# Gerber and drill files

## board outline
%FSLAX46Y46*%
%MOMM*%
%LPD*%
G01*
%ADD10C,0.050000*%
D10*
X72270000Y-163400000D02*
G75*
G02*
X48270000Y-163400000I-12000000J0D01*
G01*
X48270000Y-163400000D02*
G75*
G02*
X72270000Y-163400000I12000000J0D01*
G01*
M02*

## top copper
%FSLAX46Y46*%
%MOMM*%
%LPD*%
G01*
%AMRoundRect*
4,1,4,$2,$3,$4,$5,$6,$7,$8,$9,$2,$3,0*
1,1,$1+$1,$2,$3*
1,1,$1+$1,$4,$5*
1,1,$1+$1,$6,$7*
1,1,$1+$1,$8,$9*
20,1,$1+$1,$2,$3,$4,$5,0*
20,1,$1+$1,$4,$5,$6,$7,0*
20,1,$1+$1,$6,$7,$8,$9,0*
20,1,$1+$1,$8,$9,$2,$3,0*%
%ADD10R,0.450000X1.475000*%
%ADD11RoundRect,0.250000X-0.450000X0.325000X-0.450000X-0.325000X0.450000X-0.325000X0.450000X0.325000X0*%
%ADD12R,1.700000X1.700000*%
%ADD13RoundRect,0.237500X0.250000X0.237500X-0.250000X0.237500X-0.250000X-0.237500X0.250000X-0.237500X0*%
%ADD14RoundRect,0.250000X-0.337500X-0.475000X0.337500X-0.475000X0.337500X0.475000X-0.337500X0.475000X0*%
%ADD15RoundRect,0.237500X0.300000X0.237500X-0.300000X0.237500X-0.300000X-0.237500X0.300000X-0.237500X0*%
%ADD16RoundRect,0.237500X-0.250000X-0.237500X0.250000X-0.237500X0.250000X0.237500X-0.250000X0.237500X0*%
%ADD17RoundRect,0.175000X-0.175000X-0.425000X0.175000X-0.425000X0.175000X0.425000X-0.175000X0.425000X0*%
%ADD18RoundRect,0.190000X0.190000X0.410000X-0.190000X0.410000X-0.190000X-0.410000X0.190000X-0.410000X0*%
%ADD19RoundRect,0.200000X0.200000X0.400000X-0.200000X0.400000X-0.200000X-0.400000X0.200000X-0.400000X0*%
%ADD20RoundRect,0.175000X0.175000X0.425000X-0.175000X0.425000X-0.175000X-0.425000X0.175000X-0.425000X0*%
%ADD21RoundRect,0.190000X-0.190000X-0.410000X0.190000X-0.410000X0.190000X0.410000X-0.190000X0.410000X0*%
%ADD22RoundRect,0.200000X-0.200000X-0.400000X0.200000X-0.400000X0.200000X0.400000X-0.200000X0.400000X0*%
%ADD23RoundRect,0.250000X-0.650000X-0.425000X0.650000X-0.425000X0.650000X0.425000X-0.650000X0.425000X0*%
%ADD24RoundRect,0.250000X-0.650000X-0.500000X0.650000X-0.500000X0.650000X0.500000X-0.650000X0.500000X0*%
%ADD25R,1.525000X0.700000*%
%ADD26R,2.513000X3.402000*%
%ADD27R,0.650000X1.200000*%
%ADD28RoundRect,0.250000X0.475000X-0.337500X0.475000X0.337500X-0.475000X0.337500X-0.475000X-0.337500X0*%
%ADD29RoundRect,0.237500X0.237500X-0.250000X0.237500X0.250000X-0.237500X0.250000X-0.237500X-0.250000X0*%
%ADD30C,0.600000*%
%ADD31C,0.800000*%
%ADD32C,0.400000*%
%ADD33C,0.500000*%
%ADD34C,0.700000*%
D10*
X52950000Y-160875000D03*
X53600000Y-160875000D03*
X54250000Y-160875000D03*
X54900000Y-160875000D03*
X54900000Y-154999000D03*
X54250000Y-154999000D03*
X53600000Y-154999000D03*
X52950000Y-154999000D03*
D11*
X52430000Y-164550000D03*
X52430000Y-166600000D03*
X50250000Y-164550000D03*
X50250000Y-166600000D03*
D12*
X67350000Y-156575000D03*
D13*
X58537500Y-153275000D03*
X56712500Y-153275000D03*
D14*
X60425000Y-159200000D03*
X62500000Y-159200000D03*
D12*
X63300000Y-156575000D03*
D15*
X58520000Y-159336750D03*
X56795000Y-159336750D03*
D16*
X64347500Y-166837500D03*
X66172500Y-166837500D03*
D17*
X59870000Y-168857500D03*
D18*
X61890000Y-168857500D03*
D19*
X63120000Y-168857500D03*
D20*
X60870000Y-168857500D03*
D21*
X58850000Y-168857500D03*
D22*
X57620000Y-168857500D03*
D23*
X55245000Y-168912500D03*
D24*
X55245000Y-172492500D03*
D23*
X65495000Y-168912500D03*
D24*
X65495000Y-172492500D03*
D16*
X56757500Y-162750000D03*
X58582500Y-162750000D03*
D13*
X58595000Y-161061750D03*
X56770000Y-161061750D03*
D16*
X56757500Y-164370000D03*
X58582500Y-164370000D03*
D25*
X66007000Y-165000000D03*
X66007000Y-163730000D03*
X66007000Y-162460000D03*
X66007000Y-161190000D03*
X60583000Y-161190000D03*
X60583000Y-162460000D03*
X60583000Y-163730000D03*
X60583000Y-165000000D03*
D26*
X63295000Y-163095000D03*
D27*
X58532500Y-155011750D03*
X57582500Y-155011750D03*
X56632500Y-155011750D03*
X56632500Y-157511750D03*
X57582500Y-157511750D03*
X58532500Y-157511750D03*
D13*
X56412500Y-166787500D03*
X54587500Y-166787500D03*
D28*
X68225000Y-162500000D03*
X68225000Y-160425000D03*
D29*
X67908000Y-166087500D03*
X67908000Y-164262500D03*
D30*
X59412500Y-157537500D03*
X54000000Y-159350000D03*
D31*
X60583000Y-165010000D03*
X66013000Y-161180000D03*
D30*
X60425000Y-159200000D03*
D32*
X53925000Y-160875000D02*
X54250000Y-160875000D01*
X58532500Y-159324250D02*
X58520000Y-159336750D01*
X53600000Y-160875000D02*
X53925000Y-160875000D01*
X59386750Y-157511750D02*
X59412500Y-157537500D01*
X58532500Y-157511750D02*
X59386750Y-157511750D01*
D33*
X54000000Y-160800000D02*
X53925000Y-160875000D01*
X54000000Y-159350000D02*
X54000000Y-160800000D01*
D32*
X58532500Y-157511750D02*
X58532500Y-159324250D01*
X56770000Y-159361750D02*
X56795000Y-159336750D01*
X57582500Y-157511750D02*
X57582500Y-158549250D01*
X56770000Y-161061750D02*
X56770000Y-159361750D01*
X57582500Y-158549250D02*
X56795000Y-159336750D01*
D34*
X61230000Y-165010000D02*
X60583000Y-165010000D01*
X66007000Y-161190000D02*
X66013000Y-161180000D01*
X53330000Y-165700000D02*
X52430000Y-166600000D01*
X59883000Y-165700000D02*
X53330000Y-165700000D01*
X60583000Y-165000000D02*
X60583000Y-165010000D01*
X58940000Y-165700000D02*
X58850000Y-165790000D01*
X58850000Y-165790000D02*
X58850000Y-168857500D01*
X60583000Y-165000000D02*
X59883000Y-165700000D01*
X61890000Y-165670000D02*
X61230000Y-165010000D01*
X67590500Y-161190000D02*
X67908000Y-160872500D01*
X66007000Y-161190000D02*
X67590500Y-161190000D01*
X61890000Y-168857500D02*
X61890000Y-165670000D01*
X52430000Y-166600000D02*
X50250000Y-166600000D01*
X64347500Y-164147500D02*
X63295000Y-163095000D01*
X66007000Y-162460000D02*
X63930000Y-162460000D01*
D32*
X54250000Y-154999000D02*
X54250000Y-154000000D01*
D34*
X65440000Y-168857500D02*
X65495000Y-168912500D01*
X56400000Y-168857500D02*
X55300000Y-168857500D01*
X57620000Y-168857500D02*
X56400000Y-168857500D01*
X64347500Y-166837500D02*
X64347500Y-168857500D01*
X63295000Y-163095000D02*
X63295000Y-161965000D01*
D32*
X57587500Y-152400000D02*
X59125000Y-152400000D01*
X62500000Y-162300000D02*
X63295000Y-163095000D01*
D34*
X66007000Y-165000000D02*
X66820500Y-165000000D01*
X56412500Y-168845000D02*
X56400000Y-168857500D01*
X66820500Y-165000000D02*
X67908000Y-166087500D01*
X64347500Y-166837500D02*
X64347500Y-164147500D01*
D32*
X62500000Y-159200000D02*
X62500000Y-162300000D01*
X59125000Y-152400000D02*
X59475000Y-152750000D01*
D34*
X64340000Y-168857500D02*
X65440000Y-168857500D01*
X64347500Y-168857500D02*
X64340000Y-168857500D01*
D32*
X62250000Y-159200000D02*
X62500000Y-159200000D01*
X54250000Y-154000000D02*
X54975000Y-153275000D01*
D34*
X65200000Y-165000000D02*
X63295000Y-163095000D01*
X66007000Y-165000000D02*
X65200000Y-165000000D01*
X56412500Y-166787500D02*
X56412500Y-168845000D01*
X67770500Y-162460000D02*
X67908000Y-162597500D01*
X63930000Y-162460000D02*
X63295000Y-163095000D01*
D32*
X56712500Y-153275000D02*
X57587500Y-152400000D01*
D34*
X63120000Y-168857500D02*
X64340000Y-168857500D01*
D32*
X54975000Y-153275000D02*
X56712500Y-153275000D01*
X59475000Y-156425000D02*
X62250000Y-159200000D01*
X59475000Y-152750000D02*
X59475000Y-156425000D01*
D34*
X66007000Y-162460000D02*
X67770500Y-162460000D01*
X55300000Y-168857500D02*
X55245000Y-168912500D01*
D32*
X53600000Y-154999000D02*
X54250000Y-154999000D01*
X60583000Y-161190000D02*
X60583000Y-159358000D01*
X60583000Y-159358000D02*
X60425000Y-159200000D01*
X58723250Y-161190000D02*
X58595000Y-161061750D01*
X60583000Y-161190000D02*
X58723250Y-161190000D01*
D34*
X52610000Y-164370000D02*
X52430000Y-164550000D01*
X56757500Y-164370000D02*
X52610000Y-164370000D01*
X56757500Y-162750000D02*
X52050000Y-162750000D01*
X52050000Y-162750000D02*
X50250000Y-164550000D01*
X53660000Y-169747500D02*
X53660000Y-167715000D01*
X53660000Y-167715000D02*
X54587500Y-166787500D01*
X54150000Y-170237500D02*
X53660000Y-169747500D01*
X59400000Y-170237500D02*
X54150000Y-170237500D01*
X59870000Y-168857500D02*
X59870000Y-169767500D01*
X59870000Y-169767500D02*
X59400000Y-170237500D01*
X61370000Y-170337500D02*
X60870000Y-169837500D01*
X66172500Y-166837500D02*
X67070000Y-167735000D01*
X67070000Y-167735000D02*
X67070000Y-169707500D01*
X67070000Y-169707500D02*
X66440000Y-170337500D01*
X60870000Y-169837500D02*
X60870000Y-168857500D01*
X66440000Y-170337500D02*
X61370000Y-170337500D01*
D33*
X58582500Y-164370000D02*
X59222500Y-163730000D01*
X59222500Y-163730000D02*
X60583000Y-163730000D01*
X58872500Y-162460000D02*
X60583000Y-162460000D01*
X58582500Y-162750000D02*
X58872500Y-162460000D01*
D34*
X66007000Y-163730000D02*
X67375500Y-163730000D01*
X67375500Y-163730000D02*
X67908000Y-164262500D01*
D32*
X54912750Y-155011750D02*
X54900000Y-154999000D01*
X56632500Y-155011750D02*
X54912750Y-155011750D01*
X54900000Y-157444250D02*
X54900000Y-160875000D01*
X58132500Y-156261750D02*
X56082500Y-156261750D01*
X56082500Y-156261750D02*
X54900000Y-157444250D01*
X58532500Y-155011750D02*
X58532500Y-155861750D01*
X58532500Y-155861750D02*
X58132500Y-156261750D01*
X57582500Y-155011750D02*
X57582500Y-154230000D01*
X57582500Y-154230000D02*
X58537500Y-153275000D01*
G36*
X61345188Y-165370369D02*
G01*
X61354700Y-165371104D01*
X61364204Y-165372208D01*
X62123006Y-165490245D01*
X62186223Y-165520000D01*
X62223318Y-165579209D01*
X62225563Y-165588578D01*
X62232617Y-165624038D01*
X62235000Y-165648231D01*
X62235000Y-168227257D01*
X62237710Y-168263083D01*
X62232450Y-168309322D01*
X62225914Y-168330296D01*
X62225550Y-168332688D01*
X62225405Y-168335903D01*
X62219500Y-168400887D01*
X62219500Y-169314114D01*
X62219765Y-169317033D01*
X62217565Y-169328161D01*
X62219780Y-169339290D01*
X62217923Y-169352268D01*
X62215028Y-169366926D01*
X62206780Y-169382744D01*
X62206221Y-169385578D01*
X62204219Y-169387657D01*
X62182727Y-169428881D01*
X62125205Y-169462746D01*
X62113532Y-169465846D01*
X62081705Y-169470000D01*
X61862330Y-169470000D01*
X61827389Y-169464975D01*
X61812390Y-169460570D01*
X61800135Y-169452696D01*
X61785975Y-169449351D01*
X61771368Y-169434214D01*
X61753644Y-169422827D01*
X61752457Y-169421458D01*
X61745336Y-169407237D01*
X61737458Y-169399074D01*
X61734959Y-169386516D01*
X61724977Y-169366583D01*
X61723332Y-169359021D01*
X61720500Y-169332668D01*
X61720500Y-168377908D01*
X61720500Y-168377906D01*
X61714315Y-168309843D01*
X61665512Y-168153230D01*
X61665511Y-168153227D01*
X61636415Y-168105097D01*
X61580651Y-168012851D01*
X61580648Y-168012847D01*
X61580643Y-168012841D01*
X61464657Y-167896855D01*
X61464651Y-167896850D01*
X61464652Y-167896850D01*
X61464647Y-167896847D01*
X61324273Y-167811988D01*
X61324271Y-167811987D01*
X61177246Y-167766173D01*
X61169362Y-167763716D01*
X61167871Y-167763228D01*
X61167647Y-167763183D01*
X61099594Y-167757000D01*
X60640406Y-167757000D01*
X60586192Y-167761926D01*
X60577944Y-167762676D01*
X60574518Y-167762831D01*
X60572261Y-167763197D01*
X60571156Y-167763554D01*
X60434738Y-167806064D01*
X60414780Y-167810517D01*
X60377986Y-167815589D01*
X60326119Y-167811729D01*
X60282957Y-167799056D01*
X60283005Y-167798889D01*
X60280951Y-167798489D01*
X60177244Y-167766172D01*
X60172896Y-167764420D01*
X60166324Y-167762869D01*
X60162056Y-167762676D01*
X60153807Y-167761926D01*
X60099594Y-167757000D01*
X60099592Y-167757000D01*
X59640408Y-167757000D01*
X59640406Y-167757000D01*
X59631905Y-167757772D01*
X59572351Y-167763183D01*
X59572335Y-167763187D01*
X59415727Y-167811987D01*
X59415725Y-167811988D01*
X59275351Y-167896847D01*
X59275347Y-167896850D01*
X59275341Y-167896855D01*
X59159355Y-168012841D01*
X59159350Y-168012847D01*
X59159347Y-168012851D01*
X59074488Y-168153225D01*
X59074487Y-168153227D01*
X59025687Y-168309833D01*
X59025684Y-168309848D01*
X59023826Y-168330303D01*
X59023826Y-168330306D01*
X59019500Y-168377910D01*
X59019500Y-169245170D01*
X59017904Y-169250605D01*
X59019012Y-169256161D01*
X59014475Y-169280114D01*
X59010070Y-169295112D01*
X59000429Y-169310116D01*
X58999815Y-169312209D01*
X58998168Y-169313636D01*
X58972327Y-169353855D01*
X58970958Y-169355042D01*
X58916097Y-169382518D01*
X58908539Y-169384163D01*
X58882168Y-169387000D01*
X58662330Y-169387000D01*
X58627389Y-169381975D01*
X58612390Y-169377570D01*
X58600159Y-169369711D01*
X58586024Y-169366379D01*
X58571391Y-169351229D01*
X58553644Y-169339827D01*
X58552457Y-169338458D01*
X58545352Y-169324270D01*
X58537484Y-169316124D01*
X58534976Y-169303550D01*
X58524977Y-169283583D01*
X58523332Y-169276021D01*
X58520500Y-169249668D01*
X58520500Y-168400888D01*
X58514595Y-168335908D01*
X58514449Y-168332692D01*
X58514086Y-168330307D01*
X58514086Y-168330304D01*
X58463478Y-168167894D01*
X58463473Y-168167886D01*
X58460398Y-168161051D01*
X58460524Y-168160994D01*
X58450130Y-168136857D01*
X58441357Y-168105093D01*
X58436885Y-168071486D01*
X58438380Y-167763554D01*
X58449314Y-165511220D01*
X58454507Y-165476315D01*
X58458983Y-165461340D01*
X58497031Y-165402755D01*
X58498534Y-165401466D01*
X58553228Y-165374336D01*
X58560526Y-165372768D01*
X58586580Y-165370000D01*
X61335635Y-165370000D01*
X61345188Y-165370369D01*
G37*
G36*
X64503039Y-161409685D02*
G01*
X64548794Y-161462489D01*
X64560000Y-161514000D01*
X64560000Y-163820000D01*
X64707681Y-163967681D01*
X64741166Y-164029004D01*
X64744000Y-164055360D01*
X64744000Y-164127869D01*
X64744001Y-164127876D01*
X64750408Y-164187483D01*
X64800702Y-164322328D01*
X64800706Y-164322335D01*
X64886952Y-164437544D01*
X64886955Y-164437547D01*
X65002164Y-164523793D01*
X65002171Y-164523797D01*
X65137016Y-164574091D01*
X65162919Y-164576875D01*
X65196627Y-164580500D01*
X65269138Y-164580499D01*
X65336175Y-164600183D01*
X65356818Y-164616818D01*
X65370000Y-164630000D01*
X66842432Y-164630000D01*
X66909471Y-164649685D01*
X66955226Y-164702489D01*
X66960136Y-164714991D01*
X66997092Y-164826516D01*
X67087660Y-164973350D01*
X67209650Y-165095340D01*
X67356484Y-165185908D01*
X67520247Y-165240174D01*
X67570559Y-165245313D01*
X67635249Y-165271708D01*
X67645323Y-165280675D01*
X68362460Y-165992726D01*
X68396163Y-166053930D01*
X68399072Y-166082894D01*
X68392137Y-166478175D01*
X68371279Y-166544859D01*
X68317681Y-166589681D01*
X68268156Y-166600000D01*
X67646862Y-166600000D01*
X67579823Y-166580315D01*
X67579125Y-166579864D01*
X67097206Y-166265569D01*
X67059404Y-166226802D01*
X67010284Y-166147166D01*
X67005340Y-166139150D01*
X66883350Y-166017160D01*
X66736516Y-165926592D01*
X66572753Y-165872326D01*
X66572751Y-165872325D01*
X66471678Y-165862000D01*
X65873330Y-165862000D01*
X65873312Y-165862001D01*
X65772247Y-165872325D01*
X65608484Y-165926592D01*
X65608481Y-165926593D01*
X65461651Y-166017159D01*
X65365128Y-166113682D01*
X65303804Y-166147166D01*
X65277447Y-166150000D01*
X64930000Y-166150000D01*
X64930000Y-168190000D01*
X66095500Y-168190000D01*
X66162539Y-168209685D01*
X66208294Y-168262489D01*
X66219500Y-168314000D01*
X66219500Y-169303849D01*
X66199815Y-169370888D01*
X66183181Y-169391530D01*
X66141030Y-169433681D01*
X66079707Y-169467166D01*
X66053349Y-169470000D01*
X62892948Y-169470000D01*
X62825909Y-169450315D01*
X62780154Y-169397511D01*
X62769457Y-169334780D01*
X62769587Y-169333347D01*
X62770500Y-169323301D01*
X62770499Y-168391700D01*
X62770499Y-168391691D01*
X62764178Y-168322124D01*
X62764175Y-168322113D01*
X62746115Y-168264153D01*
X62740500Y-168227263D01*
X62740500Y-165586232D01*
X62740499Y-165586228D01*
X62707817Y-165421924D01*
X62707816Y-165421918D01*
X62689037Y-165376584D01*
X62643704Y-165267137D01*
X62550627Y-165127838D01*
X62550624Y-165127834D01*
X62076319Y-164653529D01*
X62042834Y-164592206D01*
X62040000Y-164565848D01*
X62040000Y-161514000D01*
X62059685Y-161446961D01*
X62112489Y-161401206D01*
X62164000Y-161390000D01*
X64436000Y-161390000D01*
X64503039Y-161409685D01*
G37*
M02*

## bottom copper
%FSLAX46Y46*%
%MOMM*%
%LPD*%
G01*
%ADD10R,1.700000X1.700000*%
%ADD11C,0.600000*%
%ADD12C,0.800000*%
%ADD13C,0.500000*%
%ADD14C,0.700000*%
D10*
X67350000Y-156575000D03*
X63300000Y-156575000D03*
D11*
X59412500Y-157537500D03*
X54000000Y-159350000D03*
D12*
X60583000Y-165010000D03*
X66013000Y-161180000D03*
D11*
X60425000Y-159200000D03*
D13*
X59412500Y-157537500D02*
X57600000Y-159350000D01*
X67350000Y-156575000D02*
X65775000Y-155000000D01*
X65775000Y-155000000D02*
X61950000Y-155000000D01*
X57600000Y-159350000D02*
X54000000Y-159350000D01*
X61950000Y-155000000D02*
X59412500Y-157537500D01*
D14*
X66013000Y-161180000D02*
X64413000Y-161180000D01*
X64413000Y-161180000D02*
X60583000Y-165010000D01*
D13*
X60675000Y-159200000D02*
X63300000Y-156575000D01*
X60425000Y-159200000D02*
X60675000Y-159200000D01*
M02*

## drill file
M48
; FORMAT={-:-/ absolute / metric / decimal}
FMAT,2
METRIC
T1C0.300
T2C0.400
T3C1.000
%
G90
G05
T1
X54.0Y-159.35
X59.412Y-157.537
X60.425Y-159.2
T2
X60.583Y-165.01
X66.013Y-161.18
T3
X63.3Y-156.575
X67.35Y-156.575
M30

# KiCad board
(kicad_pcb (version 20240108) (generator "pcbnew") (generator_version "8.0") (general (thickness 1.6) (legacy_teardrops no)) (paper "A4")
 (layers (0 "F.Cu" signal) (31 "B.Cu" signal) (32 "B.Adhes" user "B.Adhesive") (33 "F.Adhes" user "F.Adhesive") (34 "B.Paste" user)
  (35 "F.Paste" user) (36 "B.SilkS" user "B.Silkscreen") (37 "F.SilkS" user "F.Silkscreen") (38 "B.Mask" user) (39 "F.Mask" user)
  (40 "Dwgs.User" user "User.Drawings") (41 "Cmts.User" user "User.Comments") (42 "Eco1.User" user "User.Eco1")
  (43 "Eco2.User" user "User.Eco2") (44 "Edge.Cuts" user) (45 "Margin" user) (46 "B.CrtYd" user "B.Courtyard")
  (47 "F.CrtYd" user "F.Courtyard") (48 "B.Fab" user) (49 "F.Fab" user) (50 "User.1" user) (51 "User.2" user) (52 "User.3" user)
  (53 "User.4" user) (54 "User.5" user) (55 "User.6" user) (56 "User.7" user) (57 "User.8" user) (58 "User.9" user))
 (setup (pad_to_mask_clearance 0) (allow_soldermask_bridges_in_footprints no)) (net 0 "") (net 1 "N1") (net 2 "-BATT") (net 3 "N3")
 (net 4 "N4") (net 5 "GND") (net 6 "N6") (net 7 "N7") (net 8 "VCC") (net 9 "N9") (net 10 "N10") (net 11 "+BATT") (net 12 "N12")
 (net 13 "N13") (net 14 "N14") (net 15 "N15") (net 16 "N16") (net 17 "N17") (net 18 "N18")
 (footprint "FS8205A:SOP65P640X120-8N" (layer "F.Cu") (at 53.925 157.937 90)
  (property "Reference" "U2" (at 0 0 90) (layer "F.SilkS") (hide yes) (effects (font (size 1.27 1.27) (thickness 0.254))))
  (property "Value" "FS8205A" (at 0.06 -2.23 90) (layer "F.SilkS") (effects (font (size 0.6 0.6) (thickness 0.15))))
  (pad "1" smd rect (at -2.938 -0.975 180) (size 0.45 1.475) (layers "F.Cu" "F.Paste" "F.Mask") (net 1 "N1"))
  (pad "2" smd rect (at -2.938 -0.325 180) (size 0.45 1.475) (layers "F.Cu" "F.Paste" "F.Mask") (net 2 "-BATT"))
  (pad "3" smd rect (at -2.938 0.325 180) (size 0.45 1.475) (layers "F.Cu" "F.Paste" "F.Mask") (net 2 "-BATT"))
  (pad "4" smd rect (at -2.938 0.975 180) (size 0.45 1.475) (layers "F.Cu" "F.Paste" "F.Mask") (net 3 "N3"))
  (pad "5" smd rect (at 2.938 0.975 180) (size 0.45 1.475) (layers "F.Cu" "F.Paste" "F.Mask") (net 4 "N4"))
  (pad "6" smd rect (at 2.938 0.325 180) (size 0.45 1.475) (layers "F.Cu" "F.Paste" "F.Mask") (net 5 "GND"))
  (pad "7" smd rect (at 2.938 -0.325 180) (size 0.45 1.475) (layers "F.Cu" "F.Paste" "F.Mask") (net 5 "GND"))
  (pad "8" smd rect (at 2.938 -0.975 180) (size 0.45 1.475) (layers "F.Cu" "F.Paste" "F.Mask") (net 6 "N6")))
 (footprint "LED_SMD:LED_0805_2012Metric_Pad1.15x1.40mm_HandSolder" (layer "F.Cu") (at 52.43 165.575 -90)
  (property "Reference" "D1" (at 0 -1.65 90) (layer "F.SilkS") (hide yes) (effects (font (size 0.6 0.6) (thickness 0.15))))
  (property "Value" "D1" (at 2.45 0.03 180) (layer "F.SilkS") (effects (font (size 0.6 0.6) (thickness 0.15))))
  (pad "1" smd roundrect (at -1.025 0 270) (size 1.15 1.4) (layers "F.Cu" "F.Paste" "F.Mask") (roundrect_rratio 0.2173913043) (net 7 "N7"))
  (pad "2" smd roundrect (at 1.025 0 270) (size 1.15 1.4) (layers "F.Cu" "F.Paste" "F.Mask") (roundrect_rratio 0.2173913043) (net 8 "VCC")))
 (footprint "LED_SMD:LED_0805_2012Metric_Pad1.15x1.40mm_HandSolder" (layer "F.Cu") (at 50.25 165.575 -90)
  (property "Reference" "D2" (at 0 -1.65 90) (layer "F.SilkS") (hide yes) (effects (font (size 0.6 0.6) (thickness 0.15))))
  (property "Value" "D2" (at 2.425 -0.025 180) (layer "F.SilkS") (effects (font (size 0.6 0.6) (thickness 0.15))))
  (pad "1" smd roundrect (at -1.025 0 270) (size 1.15 1.4) (layers "F.Cu" "F.Paste" "F.Mask") (roundrect_rratio 0.2173913043) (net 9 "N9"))
  (pad "2" smd roundrect (at 1.025 0 270) (size 1.15 1.4) (layers "F.Cu" "F.Paste" "F.Mask") (roundrect_rratio 0.2173913043) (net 8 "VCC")))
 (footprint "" (layer "F.Cu") (at 67.35 156.575)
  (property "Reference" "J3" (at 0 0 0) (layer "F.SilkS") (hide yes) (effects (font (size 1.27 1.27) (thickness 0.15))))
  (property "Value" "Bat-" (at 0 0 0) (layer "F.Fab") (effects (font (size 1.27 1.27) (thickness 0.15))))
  (pad "1" thru_hole rect (at 0 0 90) (size 1.7 1.7) (drill 1) (layers "*.Cu" "*.Mask") (remove_unused_layers no) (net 2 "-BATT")))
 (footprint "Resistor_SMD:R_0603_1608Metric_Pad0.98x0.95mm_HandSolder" (layer "F.Cu") (at 57.625 153.275 180)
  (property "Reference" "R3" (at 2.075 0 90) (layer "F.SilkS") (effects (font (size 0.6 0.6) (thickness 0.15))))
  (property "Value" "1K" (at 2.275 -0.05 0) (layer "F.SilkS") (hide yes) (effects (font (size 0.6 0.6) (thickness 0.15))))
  (pad "1" smd roundrect (at -0.9125 0 180) (size 0.975 0.95) (layers "F.Cu" "F.Paste" "F.Mask") (roundrect_rratio 0.25) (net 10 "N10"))
  (pad "2" smd roundrect (at 0.9125 0 180) (size 0.975 0.95) (layers "F.Cu" "F.Paste" "F.Mask") (roundrect_rratio 0.25) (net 5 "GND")))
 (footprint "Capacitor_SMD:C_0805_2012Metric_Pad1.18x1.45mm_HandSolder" (layer "F.Cu") (at 61.4625 159.2)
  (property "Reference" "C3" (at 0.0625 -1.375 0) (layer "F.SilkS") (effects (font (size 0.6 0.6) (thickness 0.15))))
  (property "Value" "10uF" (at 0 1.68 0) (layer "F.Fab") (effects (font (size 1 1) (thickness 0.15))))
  (pad "1" smd roundrect (at -1.0375 0) (size 1.175 1.45) (layers "F.Cu" "F.Paste" "F.Mask") (roundrect_rratio 0.212766) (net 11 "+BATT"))
  (pad "2" smd roundrect (at 1.0375 0) (size 1.175 1.45) (layers "F.Cu" "F.Paste" "F.Mask") (roundrect_rratio 0.212766) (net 5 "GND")))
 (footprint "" (layer "F.Cu") (at 63.3 156.575)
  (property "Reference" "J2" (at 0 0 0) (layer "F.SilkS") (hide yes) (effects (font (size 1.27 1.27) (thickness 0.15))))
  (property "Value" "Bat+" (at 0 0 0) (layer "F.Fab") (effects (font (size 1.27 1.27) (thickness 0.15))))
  (pad "1" thru_hole rect (at 0 0 90) (size 1.7 1.7) (drill 1) (layers "*.Cu" "*.Mask") (remove_unused_layers no) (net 11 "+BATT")))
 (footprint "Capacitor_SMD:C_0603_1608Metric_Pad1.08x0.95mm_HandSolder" (layer "F.Cu") (at 57.6575 159.33675 180)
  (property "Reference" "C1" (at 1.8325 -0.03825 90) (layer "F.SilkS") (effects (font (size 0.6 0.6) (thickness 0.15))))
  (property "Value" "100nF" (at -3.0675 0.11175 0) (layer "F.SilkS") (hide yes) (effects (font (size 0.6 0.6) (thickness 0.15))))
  (pad "1" smd roundrect (at -0.8625 0 180) (size 1.075 0.95) (layers "F.Cu" "F.Paste" "F.Mask") (roundrect_rratio 0.25) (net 2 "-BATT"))
  (pad "2" smd roundrect (at 0.8625 0 180) (size 1.075 0.95) (layers "F.Cu" "F.Paste" "F.Mask") (roundrect_rratio 0.25) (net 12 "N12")))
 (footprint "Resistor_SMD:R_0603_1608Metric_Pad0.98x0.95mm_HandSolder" (layer "F.Cu") (at 65.26 166.8375)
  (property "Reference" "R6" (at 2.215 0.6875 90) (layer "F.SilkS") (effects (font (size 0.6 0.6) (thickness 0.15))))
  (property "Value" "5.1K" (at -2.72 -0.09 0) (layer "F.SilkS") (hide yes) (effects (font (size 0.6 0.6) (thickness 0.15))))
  (pad "1" smd roundrect (at -0.9125 0) (size 0.975 0.95) (layers "F.Cu" "F.Paste" "F.Mask") (roundrect_rratio 0.25) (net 5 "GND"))
  (pad "2" smd roundrect (at 0.9125 0) (size 0.975 0.95) (layers "F.Cu" "F.Paste" "F.Mask") (roundrect_rratio 0.25) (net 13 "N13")))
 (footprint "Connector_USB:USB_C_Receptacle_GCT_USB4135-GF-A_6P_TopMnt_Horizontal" (layer "F.Cu") (at 60.37 171.89)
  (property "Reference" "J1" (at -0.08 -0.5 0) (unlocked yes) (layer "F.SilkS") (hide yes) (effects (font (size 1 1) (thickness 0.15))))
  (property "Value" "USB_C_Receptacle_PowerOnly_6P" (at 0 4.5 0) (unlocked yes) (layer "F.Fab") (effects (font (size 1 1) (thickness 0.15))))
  (pad "A5" smd roundrect (at -0.5 -3.0325) (size 0.7 1.2) (layers "F.Cu" "F.Paste" "F.Mask") (roundrect_rratio 0.25) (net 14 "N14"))
  (pad "A9" smd roundrect (at 1.52 -3.0325 180) (size 0.76 1.2) (layers "F.Cu" "F.Paste" "F.Mask") (roundrect_rratio 0.25) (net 8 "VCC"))
  (pad "A12" smd roundrect (at 2.75 -3.0325 180) (size 0.8 1.2) (layers "F.Cu" "F.Paste" "F.Mask") (roundrect_rratio 0.25) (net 5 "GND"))
  (pad "B5" smd roundrect (at 0.5 -3.0325 180) (size 0.7 1.2) (layers "F.Cu" "F.Paste" "F.Mask") (roundrect_rratio 0.25) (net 13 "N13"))
  (pad "B9" smd roundrect (at -1.52 -3.0325) (size 0.76 1.2) (layers "F.Cu" "F.Paste" "F.Mask") (roundrect_rratio 0.25) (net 8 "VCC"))
  (pad "B12" smd roundrect (at -2.75 -3.0325) (size 0.8 1.2) (layers "F.Cu" "F.Paste" "F.Mask") (roundrect_rratio 0.25) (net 5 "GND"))
  (pad "S1" smd roundrect (at -5.125 -2.9775) (size 1.8 1.35) (layers "F.Cu" "F.Paste" "F.Mask") (roundrect_rratio 0.1851851852)
   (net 5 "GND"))
  (pad "S1" smd roundrect (at -5.125 0.6025) (size 1.8 1.5) (layers "F.Cu" "F.Paste" "F.Mask") (roundrect_rratio 0.1666666667) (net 5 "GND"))
  (pad "S1" smd roundrect (at 5.125 -2.9775) (size 1.8 1.35) (layers "F.Cu" "F.Paste" "F.Mask") (roundrect_rratio 0.1851851852)
   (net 5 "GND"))
  (pad "S1" smd roundrect (at 5.125 0.6025) (size 1.8 1.5) (layers "F.Cu" "F.Paste" "F.Mask") (roundrect_rratio 0.1666666667) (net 5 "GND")))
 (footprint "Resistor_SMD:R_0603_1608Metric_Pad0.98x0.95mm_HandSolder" (layer "F.Cu") (at 57.67 162.75)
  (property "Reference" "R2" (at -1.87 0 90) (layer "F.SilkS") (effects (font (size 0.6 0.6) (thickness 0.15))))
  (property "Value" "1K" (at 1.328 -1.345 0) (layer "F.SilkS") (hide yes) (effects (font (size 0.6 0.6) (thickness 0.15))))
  (pad "1" smd roundrect (at -0.9125 0) (size 0.975 0.95) (layers "F.Cu" "F.Paste" "F.Mask") (roundrect_rratio 0.25) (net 9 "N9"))
  (pad "2" smd roundrect (at 0.9125 0) (size 0.975 0.95) (layers "F.Cu" "F.Paste" "F.Mask") (roundrect_rratio 0.25) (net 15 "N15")))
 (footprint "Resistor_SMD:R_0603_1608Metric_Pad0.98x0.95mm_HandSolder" (layer "F.Cu") (at 57.6825 161.06175 180)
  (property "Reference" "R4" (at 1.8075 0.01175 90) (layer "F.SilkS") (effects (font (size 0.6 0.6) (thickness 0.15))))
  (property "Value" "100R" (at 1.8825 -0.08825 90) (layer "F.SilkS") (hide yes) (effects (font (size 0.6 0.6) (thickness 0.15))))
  (pad "1" smd roundrect (at -0.9125 0 180) (size 0.975 0.95) (layers "F.Cu" "F.Paste" "F.Mask") (roundrect_rratio 0.25) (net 11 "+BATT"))
  (pad "2" smd roundrect (at 0.9125 0 180) (size 0.975 0.95) (layers "F.Cu" "F.Paste" "F.Mask") (roundrect_rratio 0.25) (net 12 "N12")))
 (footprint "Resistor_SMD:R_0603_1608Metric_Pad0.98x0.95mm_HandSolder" (layer "F.Cu") (at 57.67 164.37)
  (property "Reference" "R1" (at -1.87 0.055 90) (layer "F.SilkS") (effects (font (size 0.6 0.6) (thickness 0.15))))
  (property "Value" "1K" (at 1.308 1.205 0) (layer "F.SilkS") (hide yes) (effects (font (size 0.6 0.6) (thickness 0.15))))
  (pad "1" smd roundrect (at -0.9125 0) (size 0.975 0.95) (layers "F.Cu" "F.Paste" "F.Mask") (roundrect_rratio 0.25) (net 7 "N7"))
  (pad "2" smd roundrect (at 0.9125 0) (size 0.975 0.95) (layers "F.Cu" "F.Paste" "F.Mask") (roundrect_rratio 0.25) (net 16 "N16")))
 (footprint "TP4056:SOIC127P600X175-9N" (layer "F.Cu") (at 63.295 163.095 180)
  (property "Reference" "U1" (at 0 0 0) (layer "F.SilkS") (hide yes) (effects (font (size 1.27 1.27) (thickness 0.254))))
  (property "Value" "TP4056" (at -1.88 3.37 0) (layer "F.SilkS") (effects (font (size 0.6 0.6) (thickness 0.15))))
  (pad "1" smd rect (at -2.712 -1.905 270) (size 0.7 1.525) (layers "F.Cu" "F.Paste" "F.Mask") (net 5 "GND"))
  (pad "2" smd rect (at -2.712 -0.635 270) (size 0.7 1.525) (layers "F.Cu" "F.Paste" "F.Mask") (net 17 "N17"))
  (pad "3" smd rect (at -2.712 0.635 270) (size 0.7 1.525) (layers "F.Cu" "F.Paste" "F.Mask") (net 5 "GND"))
  (pad "4" smd rect (at -2.712 1.905 270) (size 0.7 1.525) (layers "F.Cu" "F.Paste" "F.Mask") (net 8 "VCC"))
  (pad "5" smd rect (at 2.712 1.905 270) (size 0.7 1.525) (layers "F.Cu" "F.Paste" "F.Mask") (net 11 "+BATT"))
  (pad "6" smd rect (at 2.712 0.635 270) (size 0.7 1.525) (layers "F.Cu" "F.Paste" "F.Mask") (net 15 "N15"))
  (pad "7" smd rect (at 2.712 -0.635 270) (size 0.7 1.525) (layers "F.Cu" "F.Paste" "F.Mask") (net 16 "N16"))
  (pad "8" smd rect (at 2.712 -1.905 270) (size 0.7 1.525) (layers "F.Cu" "F.Paste" "F.Mask") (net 8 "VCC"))
  (pad "9" smd rect (at 0 0 180) (size 2.513 3.402) (layers "F.Cu" "F.Paste" "F.Mask") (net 5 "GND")))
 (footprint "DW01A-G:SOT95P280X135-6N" (layer "F.Cu") (at 57.5825 156.26175 -90)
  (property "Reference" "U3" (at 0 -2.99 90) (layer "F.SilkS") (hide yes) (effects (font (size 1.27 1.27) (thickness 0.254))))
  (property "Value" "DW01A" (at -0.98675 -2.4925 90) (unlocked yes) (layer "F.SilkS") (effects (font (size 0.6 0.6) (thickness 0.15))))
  (pad "1" smd rect (at -1.25 -0.95) (size 0.65 1.2) (layers "F.Cu" "F.Paste" "F.Mask") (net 3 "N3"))
  (pad "2" smd rect (at -1.25 0) (size 0.65 1.2) (layers "F.Cu" "F.Paste" "F.Mask") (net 10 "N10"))
  (pad "3" smd rect (at -1.25 0.95) (size 0.65 1.2) (layers "F.Cu" "F.Paste" "F.Mask") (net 4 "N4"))
  (pad "4" smd rect (at 1.25 0.95) (size 0.65 1.2) (layers "F.Cu" "F.Paste" "F.Mask") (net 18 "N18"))
  (pad "5" smd rect (at 1.25 0) (size 0.65 1.2) (layers "F.Cu" "F.Paste" "F.Mask") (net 12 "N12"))
  (pad "6" smd rect (at 1.25 -0.95) (size 0.65 1.2) (layers "F.Cu" "F.Paste" "F.Mask") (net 2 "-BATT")))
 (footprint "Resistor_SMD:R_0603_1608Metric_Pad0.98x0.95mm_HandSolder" (layer "F.Cu") (at 55.5 166.7875 180)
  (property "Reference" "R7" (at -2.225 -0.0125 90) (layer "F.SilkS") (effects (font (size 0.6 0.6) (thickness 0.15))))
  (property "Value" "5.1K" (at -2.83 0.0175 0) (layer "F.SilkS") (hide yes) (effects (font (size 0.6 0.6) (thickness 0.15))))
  (pad "1" smd roundrect (at -0.9125 0 180) (size 0.975 0.95) (layers "F.Cu" "F.Paste" "F.Mask") (roundrect_rratio 0.25) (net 5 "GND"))
  (pad "2" smd roundrect (at 0.9125 0 180) (size 0.975 0.95) (layers "F.Cu" "F.Paste" "F.Mask") (roundrect_rratio 0.25) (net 14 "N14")))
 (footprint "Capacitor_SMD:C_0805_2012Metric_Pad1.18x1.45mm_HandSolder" (layer "F.Cu") (at 68.225 161.4625 90)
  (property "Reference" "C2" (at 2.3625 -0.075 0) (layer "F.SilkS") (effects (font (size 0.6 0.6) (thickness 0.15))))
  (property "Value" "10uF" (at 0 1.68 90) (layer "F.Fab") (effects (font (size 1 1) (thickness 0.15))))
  (pad "1" smd roundrect (at -1.0375 0 90) (size 1.175 1.45) (layers "F.Cu" "F.Paste" "F.Mask") (roundrect_rratio 0.212766) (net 5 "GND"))
  (pad "2" smd roundrect (at 1.0375 0 90) (size 1.175 1.45) (layers "F.Cu" "F.Paste" "F.Mask") (roundrect_rratio 0.212766) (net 8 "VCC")))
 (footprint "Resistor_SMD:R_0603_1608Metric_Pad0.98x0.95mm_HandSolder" (layer "F.Cu") (at 67.908 165.175 90)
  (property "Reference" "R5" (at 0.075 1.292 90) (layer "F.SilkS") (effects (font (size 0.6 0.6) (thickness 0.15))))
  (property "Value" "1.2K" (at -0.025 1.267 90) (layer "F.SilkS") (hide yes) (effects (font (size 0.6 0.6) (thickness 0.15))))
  (pad "1" smd roundrect (at -0.9125 0 90) (size 0.975 0.95) (layers "F.Cu" "F.Paste" "F.Mask") (roundrect_rratio 0.25) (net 5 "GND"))
  (pad "2" smd roundrect (at 0.9125 0 90) (size 0.975 0.95) (layers "F.Cu" "F.Paste" "F.Mask") (roundrect_rratio 0.25) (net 17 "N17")))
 (gr_circle (center 60.27 163.4) (end 72.27 163.4) (stroke (width 0.05) (type default)) (fill none) (layer "Edge.Cuts"))
 (segment (start 53.925 160.875) (end 54.25 160.875) (width 0.4) (layer "F.Cu") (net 2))
 (segment (start 58.5325 159.32425) (end 58.52 159.33675) (width 0.4) (layer "F.Cu") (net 2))
 (segment (start 53.6 160.875) (end 53.925 160.875) (width 0.4) (layer "F.Cu") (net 2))
 (segment (start 59.38675 157.51175) (end 59.4125 157.5375) (width 0.4) (layer "F.Cu") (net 2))
 (segment (start 58.5325 157.51175) (end 59.38675 157.51175) (width 0.4) (layer "F.Cu") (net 2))
 (segment (start 54 160.8) (end 53.925 160.875) (width 0.5) (layer "F.Cu") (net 2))
 (segment (start 54 159.35) (end 54 160.8) (width 0.5) (layer "F.Cu") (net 2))
 (segment (start 58.5325 157.51175) (end 58.5325 159.32425) (width 0.4) (layer "F.Cu") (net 2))
 (via (at 59.4125 157.5375) (size 0.6) (drill 0.3) (layers "F.Cu" "B.Cu") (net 2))
 (via (at 54 159.35) (size 0.6) (drill 0.3) (layers "F.Cu" "B.Cu") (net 2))
 (segment (start 59.4125 157.5375) (end 57.6 159.35) (width 0.5) (layer "B.Cu") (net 2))
 (segment (start 67.35 156.575) (end 65.775 155) (width 0.5) (layer "B.Cu") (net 2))
 (segment (start 65.775 155) (end 61.95 155) (width 0.5) (layer "B.Cu") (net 2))
 (segment (start 57.6 159.35) (end 54 159.35) (width 0.5) (layer "B.Cu") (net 2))
 (segment (start 61.95 155) (end 59.4125 157.5375) (width 0.5) (layer "B.Cu") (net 2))
 (segment (start 56.77 159.36175) (end 56.795 159.33675) (width 0.4) (layer "F.Cu") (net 12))
 (segment (start 57.5825 157.51175) (end 57.5825 158.54925) (width 0.4) (layer "F.Cu") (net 12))
 (segment (start 56.77 161.06175) (end 56.77 159.36175) (width 0.4) (layer "F.Cu") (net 12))
 (segment (start 57.5825 158.54925) (end 56.795 159.33675) (width 0.4) (layer "F.Cu") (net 12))
 (segment (start 61.23 165.01) (end 60.583 165.01) (width 0.7) (layer "F.Cu") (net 8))
 (segment (start 66.007 161.19) (end 66.013 161.18) (width 0.7) (layer "F.Cu") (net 8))
 (segment (start 53.33 165.7) (end 52.43 166.6) (width 0.7) (layer "F.Cu") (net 8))
 (segment (start 59.883 165.7) (end 53.33 165.7) (width 0.7) (layer "F.Cu") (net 8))
 (segment (start 60.583 165) (end 60.583 165.01) (width 0.7) (layer "F.Cu") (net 8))
 (segment (start 58.94 165.7) (end 58.85 165.79) (width 0.7) (layer "F.Cu") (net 8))
 (segment (start 58.85 165.79) (end 58.85 168.8575) (width 0.7) (layer "F.Cu") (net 8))
 (segment (start 60.583 165) (end 59.883 165.7) (width 0.7) (layer "F.Cu") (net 8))
 (segment (start 61.89 165.67) (end 61.23 165.01) (width 0.7) (layer "F.Cu") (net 8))
 (segment (start 67.5905 161.19) (end 67.908 160.8725) (width 0.7) (layer "F.Cu") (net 8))
 (segment (start 66.007 161.19) (end 67.5905 161.19) (width 0.7) (layer "F.Cu") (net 8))
 (segment (start 61.89 168.8575) (end 61.89 165.67) (width 0.7) (layer "F.Cu") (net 8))
 (segment (start 52.43 166.6) (end 50.25 166.6) (width 0.7) (layer "F.Cu") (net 8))
 (via (at 60.583 165.01) (size 0.8) (drill 0.4) (layers "F.Cu" "B.Cu") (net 8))
 (via (at 66.013 161.18) (size 0.8) (drill 0.4) (layers "F.Cu" "B.Cu") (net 8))
 (segment (start 66.013 161.18) (end 64.413 161.18) (width 0.7) (layer "B.Cu") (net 8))
 (segment (start 64.413 161.18) (end 60.583 165.01) (width 0.7) (layer "B.Cu") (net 8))
 (segment (start 64.3475 164.1475) (end 63.295 163.095) (width 0.7) (layer "F.Cu") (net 5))
 (segment (start 66.007 162.46) (end 63.93 162.46) (width 0.7) (layer "F.Cu") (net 5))
 (segment (start 54.25 154.999) (end 54.25 154) (width 0.4) (layer "F.Cu") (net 5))
 (segment (start 65.44 168.8575) (end 65.495 168.9125) (width 0.7) (layer "F.Cu") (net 5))
 (segment (start 56.4 168.8575) (end 55.3 168.8575) (width 0.7) (layer "F.Cu") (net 5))
 (segment (start 57.62 168.8575) (end 56.4 168.8575) (width 0.7) (layer "F.Cu") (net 5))
 (segment (start 64.3475 166.8375) (end 64.3475 168.8575) (width 0.7) (layer "F.Cu") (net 5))
 (segment (start 63.295 163.095) (end 63.295 161.965) (width 0.7) (layer "F.Cu") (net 5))
 (segment (start 57.5875 152.4) (end 59.125 152.4) (width 0.4) (layer "F.Cu") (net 5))
 (segment (start 62.5 162.3) (end 63.295 163.095) (width 0.4) (layer "F.Cu") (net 5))
 (segment (start 66.007 165) (end 66.8205 165) (width 0.7) (layer "F.Cu") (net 5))
 (segment (start 56.4125 168.845) (end 56.4 168.8575) (width 0.7) (layer "F.Cu") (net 5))
 (segment (start 66.8205 165) (end 67.908 166.0875) (width 0.7) (layer "F.Cu") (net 5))
 (segment (start 64.3475 166.8375) (end 64.3475 164.1475) (width 0.7) (layer "F.Cu") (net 5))
 (segment (start 62.5 159.2) (end 62.5 162.3) (width 0.4) (layer "F.Cu") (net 5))
 (segment (start 59.125 152.4) (end 59.475 152.75) (width 0.4) (layer "F.Cu") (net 5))
 (segment (start 64.34 168.8575) (end 65.44 168.8575) (width 0.7) (layer "F.Cu") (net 5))
 (segment (start 64.3475 168.8575) (end 64.34 168.8575) (width 0.7) (layer "F.Cu") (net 5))
 (segment (start 62.25 159.2) (end 62.5 159.2) (width 0.4) (layer "F.Cu") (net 5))
 (segment (start 54.25 154) (end 54.975 153.275) (width 0.4) (layer "F.Cu") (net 5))
 (segment (start 65.2 165) (end 63.295 163.095) (width 0.7) (layer "F.Cu") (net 5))
 (segment (start 66.007 165) (end 65.2 165) (width 0.7) (layer "F.Cu") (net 5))
 (segment (start 56.4125 166.7875) (end 56.4125 168.845) (width 0.7) (layer "F.Cu") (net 5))
 (segment (start 67.7705 162.46) (end 67.908 162.5975) (width 0.7) (layer "F.Cu") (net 5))
 (segment (start 63.93 162.46) (end 63.295 163.095) (width 0.7) (layer "F.Cu") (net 5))
 (segment (start 56.7125 153.275) (end 57.5875 152.4) (width 0.4) (layer "F.Cu") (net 5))
 (segment (start 63.12 168.8575) (end 64.34 168.8575) (width 0.7) (layer "F.Cu") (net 5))
 (segment (start 54.975 153.275) (end 56.7125 153.275) (width 0.4) (layer "F.Cu") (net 5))
 (segment (start 59.475 156.425) (end 62.25 159.2) (width 0.4) (layer "F.Cu") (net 5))
 (segment (start 59.475 152.75) (end 59.475 156.425) (width 0.4) (layer "F.Cu") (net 5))
 (segment (start 66.007 162.46) (end 67.7705 162.46) (width 0.7) (layer "F.Cu") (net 5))
 (segment (start 55.3 168.8575) (end 55.245 168.9125) (width 0.7) (layer "F.Cu") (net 5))
 (segment (start 53.6 154.999) (end 54.25 154.999) (width 0.4) (layer "F.Cu") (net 5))
 (segment (start 60.583 161.19) (end 60.583 159.358) (width 0.4) (layer "F.Cu") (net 11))
 (segment (start 60.583 159.358) (end 60.425 159.2) (width 0.4) (layer "F.Cu") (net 11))
 (segment (start 58.72325 161.19) (end 58.595 161.06175) (width 0.4) (layer "F.Cu") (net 11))
 (segment (start 60.583 161.19) (end 58.72325 161.19) (width 0.4) (layer "F.Cu") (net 11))
 (via (at 60.425 159.2) (size 0.6) (drill 0.3) (layers "F.Cu" "B.Cu") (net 11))
 (segment (start 60.675 159.2) (end 63.3 156.575) (width 0.5) (layer "B.Cu") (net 11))
 (segment (start 60.425 159.2) (end 60.675 159.2) (width 0.5) (layer "B.Cu") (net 11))
 (segment (start 52.61 164.37) (end 52.43 164.55) (width 0.7) (layer "F.Cu") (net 7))
 (segment (start 56.7575 164.37) (end 52.61 164.37) (width 0.7) (layer "F.Cu") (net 7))
 (segment (start 56.7575 162.75) (end 52.05 162.75) (width 0.7) (layer "F.Cu") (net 9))
 (segment (start 52.05 162.75) (end 50.25 164.55) (width 0.7) (layer "F.Cu") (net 9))
 (segment (start 53.66 169.7475) (end 53.66 167.715) (width 0.7) (layer "F.Cu") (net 14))
 (segment (start 53.66 167.715) (end 54.5875 166.7875) (width 0.7) (layer "F.Cu") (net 14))
 (segment (start 54.15 170.2375) (end 53.66 169.7475) (width 0.7) (layer "F.Cu") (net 14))
 (segment (start 59.4 170.2375) (end 54.15 170.2375) (width 0.7) (layer "F.Cu") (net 14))
 (segment (start 59.87 168.8575) (end 59.87 169.7675) (width 0.7) (layer "F.Cu") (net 14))
 (segment (start 59.87 169.7675) (end 59.4 170.2375) (width 0.7) (layer "F.Cu") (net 14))
 (segment (start 61.37 170.3375) (end 60.87 169.8375) (width 0.7) (layer "F.Cu") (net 13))
 (segment (start 66.1725 166.8375) (end 67.07 167.735) (width 0.7) (layer "F.Cu") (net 13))
 (segment (start 67.07 167.735) (end 67.07 169.7075) (width 0.7) (layer "F.Cu") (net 13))
 (segment (start 67.07 169.7075) (end 66.44 170.3375) (width 0.7) (layer "F.Cu") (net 13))
 (segment (start 60.87 169.8375) (end 60.87 168.8575) (width 0.7) (layer "F.Cu") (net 13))
 (segment (start 66.44 170.3375) (end 61.37 170.3375) (width 0.7) (layer "F.Cu") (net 13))
 (segment (start 58.5825 164.37) (end 59.2225 163.73) (width 0.5) (layer "F.Cu") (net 16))
 (segment (start 59.2225 163.73) (end 60.583 163.73) (width 0.5) (layer "F.Cu") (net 16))
 (segment (start 58.8725 162.46) (end 60.583 162.46) (width 0.5) (layer "F.Cu") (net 15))
 (segment (start 58.5825 162.75) (end 58.8725 162.46) (width 0.5) (layer "F.Cu") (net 15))
 (segment (start 66.007 163.73) (end 67.3755 163.73) (width 0.7) (layer "F.Cu") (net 17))
 (segment (start 67.3755 163.73) (end 67.908 164.2625) (width 0.7) (layer "F.Cu") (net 17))
 (segment (start 54.91275 155.01175) (end 54.9 154.999) (width 0.4) (layer "F.Cu") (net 4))
 (segment (start 56.6325 155.01175) (end 54.91275 155.01175) (width 0.4) (layer "F.Cu") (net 4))
 (segment (start 54.9 157.44425) (end 54.9 160.875) (width 0.4) (layer "F.Cu") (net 3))
 (segment (start 58.1325 156.26175) (end 56.0825 156.26175) (width 0.4) (layer "F.Cu") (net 3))
 (segment (start 56.0825 156.26175) (end 54.9 157.44425) (width 0.4) (layer "F.Cu") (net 3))
 (segment (start 58.5325 155.01175) (end 58.5325 155.86175) (width 0.4) (layer "F.Cu") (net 3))
 (segment (start 58.5325 155.86175) (end 58.1325 156.26175) (width 0.4) (layer "F.Cu") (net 3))
 (segment (start 57.5825 155.01175) (end 57.5825 154.23) (width 0.4) (layer "F.Cu") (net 10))
 (segment (start 57.5825 154.23) (end 58.5375 153.275) (width 0.4) (layer "F.Cu") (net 10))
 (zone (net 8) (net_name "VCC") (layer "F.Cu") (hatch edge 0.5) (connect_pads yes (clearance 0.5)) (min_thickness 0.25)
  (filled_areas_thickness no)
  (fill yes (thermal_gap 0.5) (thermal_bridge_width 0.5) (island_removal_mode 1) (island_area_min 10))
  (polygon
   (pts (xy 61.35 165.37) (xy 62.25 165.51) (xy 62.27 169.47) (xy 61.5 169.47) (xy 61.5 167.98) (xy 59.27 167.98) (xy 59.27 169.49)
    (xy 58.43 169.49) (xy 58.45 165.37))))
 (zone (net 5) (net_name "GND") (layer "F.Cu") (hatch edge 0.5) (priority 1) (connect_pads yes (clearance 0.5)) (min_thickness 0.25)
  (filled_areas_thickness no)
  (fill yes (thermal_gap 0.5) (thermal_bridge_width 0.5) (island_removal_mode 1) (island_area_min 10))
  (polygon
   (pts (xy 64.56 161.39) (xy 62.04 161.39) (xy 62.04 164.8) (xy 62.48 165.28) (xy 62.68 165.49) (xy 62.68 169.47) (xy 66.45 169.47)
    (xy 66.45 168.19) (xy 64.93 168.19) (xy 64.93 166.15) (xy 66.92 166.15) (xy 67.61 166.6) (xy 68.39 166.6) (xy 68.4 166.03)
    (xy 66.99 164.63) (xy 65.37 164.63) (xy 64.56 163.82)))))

